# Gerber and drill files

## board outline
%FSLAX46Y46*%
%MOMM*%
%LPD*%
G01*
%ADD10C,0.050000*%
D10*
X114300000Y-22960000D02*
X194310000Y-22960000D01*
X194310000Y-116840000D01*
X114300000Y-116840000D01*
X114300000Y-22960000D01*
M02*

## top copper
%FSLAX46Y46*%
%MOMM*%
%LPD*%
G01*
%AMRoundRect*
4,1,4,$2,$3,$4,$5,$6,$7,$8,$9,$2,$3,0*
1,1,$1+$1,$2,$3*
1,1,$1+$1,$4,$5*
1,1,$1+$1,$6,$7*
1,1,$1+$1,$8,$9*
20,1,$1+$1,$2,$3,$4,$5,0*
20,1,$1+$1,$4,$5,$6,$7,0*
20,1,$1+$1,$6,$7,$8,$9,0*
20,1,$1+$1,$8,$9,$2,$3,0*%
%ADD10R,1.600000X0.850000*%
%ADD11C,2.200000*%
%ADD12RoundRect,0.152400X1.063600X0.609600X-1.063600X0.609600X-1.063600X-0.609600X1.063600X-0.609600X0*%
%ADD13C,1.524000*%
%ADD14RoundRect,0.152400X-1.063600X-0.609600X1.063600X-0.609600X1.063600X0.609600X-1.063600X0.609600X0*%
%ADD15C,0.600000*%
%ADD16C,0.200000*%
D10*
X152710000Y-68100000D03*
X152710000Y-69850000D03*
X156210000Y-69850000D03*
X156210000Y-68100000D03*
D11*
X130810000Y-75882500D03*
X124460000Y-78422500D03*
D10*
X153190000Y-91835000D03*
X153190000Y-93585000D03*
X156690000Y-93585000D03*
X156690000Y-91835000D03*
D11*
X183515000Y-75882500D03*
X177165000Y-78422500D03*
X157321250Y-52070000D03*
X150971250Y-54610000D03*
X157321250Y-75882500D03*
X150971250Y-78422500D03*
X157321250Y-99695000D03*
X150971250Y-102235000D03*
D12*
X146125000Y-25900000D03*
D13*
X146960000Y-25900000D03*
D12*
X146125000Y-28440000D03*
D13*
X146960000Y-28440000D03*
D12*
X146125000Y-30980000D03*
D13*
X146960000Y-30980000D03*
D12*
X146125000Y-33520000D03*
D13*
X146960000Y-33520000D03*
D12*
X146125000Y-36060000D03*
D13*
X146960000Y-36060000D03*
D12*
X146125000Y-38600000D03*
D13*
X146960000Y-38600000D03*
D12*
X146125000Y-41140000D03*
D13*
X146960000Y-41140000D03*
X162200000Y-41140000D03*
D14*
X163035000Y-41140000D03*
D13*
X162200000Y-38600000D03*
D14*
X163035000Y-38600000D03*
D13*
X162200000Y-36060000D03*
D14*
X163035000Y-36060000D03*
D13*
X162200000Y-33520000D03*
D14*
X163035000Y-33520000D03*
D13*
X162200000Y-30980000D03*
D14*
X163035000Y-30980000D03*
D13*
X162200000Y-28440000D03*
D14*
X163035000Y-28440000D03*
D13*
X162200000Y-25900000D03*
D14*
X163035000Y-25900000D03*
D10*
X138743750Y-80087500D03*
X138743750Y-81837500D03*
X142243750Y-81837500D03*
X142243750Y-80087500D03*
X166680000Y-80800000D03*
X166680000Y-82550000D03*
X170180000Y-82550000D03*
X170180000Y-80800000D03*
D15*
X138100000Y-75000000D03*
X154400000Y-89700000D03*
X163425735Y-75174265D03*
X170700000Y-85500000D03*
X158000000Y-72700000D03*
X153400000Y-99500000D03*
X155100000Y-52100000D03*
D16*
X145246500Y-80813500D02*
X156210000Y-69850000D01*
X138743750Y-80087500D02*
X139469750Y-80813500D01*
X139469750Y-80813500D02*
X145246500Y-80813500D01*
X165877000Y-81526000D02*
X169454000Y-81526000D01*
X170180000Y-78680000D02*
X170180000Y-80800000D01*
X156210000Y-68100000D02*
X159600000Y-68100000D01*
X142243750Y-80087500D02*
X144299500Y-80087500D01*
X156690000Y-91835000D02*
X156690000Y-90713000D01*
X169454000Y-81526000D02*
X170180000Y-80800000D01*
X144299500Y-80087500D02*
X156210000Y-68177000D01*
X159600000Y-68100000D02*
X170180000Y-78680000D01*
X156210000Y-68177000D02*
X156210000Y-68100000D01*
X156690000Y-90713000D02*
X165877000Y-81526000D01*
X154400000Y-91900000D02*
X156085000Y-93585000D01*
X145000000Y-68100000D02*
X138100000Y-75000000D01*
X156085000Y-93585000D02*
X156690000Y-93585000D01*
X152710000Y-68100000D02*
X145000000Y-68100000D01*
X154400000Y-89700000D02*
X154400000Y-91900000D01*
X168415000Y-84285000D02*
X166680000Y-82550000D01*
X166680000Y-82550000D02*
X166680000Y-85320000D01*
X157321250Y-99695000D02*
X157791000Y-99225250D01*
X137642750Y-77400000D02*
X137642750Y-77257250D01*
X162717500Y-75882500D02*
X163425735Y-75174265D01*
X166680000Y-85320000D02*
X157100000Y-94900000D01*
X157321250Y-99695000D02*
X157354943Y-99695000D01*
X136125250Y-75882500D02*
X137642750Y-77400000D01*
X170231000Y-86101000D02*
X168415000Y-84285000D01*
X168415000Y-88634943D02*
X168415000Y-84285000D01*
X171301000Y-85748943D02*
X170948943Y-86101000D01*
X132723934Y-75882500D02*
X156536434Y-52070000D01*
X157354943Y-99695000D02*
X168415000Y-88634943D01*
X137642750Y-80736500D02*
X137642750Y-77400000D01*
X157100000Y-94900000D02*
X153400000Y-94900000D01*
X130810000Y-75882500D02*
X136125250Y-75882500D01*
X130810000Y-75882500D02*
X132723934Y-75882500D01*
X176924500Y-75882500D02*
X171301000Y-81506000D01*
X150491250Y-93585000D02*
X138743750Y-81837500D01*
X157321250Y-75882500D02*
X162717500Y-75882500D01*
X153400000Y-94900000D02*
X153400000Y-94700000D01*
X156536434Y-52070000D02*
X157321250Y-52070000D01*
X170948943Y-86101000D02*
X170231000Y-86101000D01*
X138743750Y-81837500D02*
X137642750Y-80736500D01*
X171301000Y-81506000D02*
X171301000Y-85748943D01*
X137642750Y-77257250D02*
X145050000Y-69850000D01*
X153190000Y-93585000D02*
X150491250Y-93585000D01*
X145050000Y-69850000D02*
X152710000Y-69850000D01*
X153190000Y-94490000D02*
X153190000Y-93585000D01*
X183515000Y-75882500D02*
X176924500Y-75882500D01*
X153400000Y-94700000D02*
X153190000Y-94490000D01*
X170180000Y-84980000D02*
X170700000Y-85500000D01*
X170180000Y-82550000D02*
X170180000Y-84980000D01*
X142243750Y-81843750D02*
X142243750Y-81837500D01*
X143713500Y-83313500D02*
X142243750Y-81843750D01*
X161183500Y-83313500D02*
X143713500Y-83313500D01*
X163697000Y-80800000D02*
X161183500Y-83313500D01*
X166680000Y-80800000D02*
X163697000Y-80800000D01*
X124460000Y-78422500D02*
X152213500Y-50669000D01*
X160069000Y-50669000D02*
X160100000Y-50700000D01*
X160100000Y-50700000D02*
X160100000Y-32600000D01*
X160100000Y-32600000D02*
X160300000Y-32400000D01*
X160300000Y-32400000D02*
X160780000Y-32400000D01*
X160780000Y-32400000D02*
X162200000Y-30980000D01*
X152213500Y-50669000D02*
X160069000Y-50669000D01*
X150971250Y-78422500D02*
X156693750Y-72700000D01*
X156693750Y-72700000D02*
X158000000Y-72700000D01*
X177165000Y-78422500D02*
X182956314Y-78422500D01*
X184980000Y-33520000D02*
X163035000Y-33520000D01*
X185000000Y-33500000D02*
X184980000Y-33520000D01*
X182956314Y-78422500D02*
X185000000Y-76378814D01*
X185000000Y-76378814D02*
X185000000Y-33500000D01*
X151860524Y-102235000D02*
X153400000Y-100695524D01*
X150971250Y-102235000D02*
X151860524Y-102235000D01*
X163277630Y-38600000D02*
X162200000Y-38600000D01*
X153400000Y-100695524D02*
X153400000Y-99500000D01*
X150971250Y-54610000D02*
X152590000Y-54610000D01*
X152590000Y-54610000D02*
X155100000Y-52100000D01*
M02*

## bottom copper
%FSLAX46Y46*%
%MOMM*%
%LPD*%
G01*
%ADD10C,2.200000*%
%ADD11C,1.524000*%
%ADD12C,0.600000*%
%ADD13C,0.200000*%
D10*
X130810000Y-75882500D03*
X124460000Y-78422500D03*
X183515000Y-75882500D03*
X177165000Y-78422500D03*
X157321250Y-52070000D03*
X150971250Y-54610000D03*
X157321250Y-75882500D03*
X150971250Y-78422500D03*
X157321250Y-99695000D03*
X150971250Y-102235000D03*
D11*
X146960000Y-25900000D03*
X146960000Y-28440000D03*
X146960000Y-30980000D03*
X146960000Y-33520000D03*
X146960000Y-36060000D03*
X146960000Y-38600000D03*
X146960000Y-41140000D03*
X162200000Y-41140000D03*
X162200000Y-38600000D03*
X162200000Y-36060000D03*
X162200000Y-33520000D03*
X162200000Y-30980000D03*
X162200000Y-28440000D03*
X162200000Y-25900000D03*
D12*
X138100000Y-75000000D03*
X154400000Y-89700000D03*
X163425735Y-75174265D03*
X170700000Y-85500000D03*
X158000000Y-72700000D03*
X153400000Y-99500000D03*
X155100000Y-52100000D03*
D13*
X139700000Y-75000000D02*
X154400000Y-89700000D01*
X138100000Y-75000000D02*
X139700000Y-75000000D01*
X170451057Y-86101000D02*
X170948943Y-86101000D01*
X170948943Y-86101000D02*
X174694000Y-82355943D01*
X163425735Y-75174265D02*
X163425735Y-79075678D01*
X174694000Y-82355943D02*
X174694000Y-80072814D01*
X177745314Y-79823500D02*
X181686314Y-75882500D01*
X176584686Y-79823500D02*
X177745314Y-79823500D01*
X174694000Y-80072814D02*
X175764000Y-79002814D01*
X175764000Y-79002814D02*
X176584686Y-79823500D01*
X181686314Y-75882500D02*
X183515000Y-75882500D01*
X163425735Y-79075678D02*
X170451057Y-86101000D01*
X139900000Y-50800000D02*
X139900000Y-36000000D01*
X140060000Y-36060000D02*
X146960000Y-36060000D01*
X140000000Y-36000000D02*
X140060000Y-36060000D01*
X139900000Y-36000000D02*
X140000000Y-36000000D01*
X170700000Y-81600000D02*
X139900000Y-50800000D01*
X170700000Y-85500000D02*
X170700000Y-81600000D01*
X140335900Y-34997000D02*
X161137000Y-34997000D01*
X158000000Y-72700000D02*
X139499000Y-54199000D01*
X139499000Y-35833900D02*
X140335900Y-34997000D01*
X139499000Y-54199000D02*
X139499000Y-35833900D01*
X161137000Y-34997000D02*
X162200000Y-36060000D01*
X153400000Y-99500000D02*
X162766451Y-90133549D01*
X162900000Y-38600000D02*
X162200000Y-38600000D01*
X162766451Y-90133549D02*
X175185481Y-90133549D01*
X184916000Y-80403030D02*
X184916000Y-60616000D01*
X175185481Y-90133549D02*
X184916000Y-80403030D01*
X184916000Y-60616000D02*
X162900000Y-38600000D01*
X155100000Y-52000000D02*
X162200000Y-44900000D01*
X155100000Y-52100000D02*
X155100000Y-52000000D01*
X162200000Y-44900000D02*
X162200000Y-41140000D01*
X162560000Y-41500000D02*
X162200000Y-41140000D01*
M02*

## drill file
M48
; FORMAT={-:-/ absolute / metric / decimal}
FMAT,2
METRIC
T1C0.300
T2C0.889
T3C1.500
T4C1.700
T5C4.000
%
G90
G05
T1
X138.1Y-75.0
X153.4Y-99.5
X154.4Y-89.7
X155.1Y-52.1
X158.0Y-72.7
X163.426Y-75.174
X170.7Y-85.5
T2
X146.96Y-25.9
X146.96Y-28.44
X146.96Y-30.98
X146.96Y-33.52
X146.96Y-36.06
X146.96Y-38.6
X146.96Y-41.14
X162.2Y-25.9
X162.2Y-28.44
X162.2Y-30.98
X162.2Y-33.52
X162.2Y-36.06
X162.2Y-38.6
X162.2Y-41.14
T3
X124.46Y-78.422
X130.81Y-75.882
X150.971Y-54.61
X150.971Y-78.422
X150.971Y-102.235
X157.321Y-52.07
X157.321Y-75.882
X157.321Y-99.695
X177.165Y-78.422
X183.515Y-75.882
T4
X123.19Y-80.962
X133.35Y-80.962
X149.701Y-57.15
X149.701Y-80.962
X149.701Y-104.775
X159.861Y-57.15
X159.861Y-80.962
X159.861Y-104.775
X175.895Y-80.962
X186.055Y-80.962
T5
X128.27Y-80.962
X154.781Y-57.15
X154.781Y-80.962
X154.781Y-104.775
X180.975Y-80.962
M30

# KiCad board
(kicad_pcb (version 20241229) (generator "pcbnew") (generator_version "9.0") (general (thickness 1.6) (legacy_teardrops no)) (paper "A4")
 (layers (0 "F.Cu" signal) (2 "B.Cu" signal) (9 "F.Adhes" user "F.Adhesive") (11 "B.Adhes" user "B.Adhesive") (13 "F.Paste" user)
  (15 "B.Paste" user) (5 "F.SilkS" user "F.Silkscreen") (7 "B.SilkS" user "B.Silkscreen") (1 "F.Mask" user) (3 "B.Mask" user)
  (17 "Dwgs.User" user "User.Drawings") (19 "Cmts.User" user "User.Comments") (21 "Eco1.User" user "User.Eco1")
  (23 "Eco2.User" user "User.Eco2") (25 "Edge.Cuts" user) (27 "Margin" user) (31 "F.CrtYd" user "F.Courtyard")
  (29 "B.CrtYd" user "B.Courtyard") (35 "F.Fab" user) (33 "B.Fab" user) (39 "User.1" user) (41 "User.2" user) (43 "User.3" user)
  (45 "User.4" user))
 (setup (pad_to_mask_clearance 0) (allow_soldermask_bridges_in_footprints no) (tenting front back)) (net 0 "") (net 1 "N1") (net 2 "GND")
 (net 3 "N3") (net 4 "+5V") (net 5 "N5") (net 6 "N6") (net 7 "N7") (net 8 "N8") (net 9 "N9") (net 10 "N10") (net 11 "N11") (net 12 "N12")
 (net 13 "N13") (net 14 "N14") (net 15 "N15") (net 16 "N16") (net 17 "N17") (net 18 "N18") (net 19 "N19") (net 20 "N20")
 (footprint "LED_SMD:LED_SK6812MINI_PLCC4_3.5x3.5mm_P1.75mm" (layer "F.Cu") (at 154.46 68.975)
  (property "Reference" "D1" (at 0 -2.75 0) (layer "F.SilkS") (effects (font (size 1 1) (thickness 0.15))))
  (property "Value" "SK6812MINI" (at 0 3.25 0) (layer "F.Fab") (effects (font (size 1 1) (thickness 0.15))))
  (pad "1" smd rect (at -1.75 -0.875) (size 1.6 0.85) (layers "F.Cu" "F.Mask" "F.Paste") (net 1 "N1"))
  (pad "2" smd rect (at -1.75 0.875) (size 1.6 0.85) (layers "F.Cu" "F.Mask" "F.Paste") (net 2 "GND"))
  (pad "3" smd rect (at 1.75 0.875) (size 1.6 0.85) (layers "F.Cu" "F.Mask" "F.Paste") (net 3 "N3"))
  (pad "4" smd rect (at 1.75 -0.875) (size 1.6 0.85) (layers "F.Cu" "F.Mask" "F.Paste") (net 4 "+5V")))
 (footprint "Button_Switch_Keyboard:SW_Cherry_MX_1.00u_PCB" (layer "F.Cu") (at 130.81 75.8825)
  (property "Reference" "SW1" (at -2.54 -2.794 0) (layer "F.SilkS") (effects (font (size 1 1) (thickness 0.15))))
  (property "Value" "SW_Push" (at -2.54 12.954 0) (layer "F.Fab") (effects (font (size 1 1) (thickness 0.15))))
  (pad "" np_thru_hole circle (at -7.62 5.08) (size 1.7 1.7) (drill 1.7) (layers "*.Cu" "*.Mask"))
  (pad "" np_thru_hole circle (at -2.54 5.08) (size 4 4) (drill 4) (layers "*.Cu" "*.Mask"))
  (pad "" np_thru_hole circle (at 2.54 5.08) (size 1.7 1.7) (drill 1.7) (layers "*.Cu" "*.Mask"))
  (pad "1" thru_hole circle (at 0 0) (size 2.2 2.2) (drill 1.5) (layers "*.Cu" "*.Mask") (remove_unused_layers no) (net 2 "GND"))
  (pad "2" thru_hole circle (at -6.35 2.54) (size 2.2 2.2) (drill 1.5) (layers "*.Cu" "*.Mask") (remove_unused_layers no) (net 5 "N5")))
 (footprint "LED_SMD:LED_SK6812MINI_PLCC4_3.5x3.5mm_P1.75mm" (layer "F.Cu") (at 154.94 92.71)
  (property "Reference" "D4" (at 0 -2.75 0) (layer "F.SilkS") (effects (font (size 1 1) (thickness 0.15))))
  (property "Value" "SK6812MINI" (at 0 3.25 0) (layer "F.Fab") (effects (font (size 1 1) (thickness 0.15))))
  (pad "1" smd rect (at -1.75 -0.875) (size 1.6 0.85) (layers "F.Cu" "F.Mask" "F.Paste") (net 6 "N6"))
  (pad "2" smd rect (at -1.75 0.875) (size 1.6 0.85) (layers "F.Cu" "F.Mask" "F.Paste") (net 2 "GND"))
  (pad "3" smd rect (at 1.75 0.875) (size 1.6 0.85) (layers "F.Cu" "F.Mask" "F.Paste") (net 1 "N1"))
  (pad "4" smd rect (at 1.75 -0.875) (size 1.6 0.85) (layers "F.Cu" "F.Mask" "F.Paste") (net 4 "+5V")))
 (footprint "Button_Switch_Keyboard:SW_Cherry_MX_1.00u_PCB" (layer "F.Cu") (at 183.515 75.8825)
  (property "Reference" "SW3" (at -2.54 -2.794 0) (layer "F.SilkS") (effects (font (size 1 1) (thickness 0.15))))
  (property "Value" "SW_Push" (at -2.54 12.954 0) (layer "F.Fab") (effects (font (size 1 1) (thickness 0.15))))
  (pad "" np_thru_hole circle (at -7.62 5.08) (size 1.7 1.7) (drill 1.7) (layers "*.Cu" "*.Mask"))
  (pad "" np_thru_hole circle (at -2.54 5.08) (size 4 4) (drill 4) (layers "*.Cu" "*.Mask"))
  (pad "" np_thru_hole circle (at 2.54 5.08) (size 1.7 1.7) (drill 1.7) (layers "*.Cu" "*.Mask"))
  (pad "1" thru_hole circle (at 0 0) (size 2.2 2.2) (drill 1.5) (layers "*.Cu" "*.Mask") (remove_unused_layers no) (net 2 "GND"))
  (pad "2" thru_hole circle (at -6.35 2.54) (size 2.2 2.2) (drill 1.5) (layers "*.Cu" "*.Mask") (remove_unused_layers no) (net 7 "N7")))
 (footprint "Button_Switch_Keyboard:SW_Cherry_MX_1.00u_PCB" (layer "F.Cu") (at 157.32125 52.07)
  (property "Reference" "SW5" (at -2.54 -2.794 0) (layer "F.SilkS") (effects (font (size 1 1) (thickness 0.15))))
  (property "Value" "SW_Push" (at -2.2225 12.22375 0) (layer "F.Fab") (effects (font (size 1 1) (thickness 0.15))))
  (pad "" np_thru_hole circle (at -7.62 5.08) (size 1.7 1.7) (drill 1.7) (layers "*.Cu" "*.Mask"))
  (pad "" np_thru_hole circle (at -2.54 5.08) (size 4 4) (drill 4) (layers "*.Cu" "*.Mask"))
  (pad "" np_thru_hole circle (at 2.54 5.08) (size 1.7 1.7) (drill 1.7) (layers "*.Cu" "*.Mask"))
  (pad "1" thru_hole circle (at 0 0) (size 2.2 2.2) (drill 1.5) (layers "*.Cu" "*.Mask") (remove_unused_layers no) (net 2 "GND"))
  (pad "2" thru_hole circle (at -6.35 2.54) (size 2.2 2.2) (drill 1.5) (layers "*.Cu" "*.Mask") (remove_unused_layers no) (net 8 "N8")))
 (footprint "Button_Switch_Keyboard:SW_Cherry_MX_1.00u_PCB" (layer "F.Cu") (at 157.32125 75.8825)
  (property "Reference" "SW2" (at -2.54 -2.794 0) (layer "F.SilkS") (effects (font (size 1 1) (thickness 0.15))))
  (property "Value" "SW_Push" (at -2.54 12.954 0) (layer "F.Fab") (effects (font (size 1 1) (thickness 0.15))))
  (pad "" np_thru_hole circle (at -7.62 5.08) (size 1.7 1.7) (drill 1.7) (layers "*.Cu" "*.Mask"))
  (pad "" np_thru_hole circle (at -2.54 5.08) (size 4 4) (drill 4) (layers "*.Cu" "*.Mask"))
  (pad "" np_thru_hole circle (at 2.54 5.08) (size 1.7 1.7) (drill 1.7) (layers "*.Cu" "*.Mask"))
  (pad "1" thru_hole circle (at 0 0) (size 2.2 2.2) (drill 1.5) (layers "*.Cu" "*.Mask") (remove_unused_layers no) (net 2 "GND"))
  (pad "2" thru_hole circle (at -6.35 2.54) (size 2.2 2.2) (drill 1.5) (layers "*.Cu" "*.Mask") (remove_unused_layers no) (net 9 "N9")))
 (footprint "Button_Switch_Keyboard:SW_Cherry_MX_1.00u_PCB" (layer "F.Cu") (at 157.32125 99.695)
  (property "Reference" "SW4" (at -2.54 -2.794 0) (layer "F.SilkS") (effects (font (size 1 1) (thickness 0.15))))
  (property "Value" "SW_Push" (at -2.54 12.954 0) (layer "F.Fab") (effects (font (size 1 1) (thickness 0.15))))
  (pad "" np_thru_hole circle (at -7.62 5.08) (size 1.7 1.7) (drill 1.7) (layers "*.Cu" "*.Mask"))
  (pad "" np_thru_hole circle (at -2.54 5.08) (size 4 4) (drill 4) (layers "*.Cu" "*.Mask"))
  (pad "" np_thru_hole circle (at 2.54 5.08) (size 1.7 1.7) (drill 1.7) (layers "*.Cu" "*.Mask"))
  (pad "1" thru_hole circle (at 0 0) (size 2.2 2.2) (drill 1.5) (layers "*.Cu" "*.Mask") (remove_unused_layers no) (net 2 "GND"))
  (pad "2" thru_hole circle (at -6.35 2.54) (size 2.2 2.2) (drill 1.5) (layers "*.Cu" "*.Mask") (remove_unused_layers no) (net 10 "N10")))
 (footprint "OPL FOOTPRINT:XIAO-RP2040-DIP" (layer "F.Cu") (at 154.58 33.52)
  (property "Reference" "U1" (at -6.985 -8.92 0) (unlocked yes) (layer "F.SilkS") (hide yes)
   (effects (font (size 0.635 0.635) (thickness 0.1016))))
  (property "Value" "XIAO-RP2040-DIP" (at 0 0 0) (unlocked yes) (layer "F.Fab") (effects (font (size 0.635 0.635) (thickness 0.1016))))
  (pad "1" smd roundrect (at -8.455 -7.62 180) (size 2.432 1.524) (layers "F.Cu" "F.Mask") (roundrect_rratio 0.1) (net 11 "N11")
   (thermal_bridge_angle 45))
  (pad "1" thru_hole circle (at -7.62 -7.62 180) (size 1.524 1.524) (drill 0.889) (layers "*.Cu" "*.Mask") (remove_unused_layers no)
   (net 11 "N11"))
  (pad "2" smd roundrect (at -8.455 -5.08 180) (size 2.432 1.524) (layers "F.Cu" "F.Mask") (roundrect_rratio 0.1) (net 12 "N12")
   (thermal_bridge_angle 45))
  (pad "2" thru_hole circle (at -7.62 -5.08 180) (size 1.524 1.524) (drill 0.889) (layers "*.Cu" "*.Mask") (remove_unused_layers no)
   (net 12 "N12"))
  (pad "3" smd roundrect (at -8.455 -2.54 180) (size 2.432 1.524) (layers "F.Cu" "F.Mask") (roundrect_rratio 0.1) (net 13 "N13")
   (thermal_bridge_angle 45))
  (pad "3" thru_hole circle (at -7.62 -2.54 180) (size 1.524 1.524) (drill 0.889) (layers "*.Cu" "*.Mask") (remove_unused_layers no)
   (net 13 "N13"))
  (pad "4" smd roundrect (at -8.455 0 180) (size 2.432 1.524) (layers "F.Cu" "F.Mask") (roundrect_rratio 0.1) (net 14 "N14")
   (thermal_bridge_angle 45))
  (pad "4" thru_hole circle (at -7.62 0 180) (size 1.524 1.524) (drill 0.889) (layers "*.Cu" "*.Mask") (remove_unused_layers no)
   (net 14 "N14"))
  (pad "5" smd roundrect (at -8.455 2.54 180) (size 2.432 1.524) (layers "F.Cu" "F.Mask") (roundrect_rratio 0.1) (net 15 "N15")
   (thermal_bridge_angle 45))
  (pad "5" thru_hole circle (at -7.62 2.54 180) (size 1.524 1.524) (drill 0.889) (layers "*.Cu" "*.Mask") (remove_unused_layers no)
   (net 15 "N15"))
  (pad "6" smd roundrect (at -8.455 5.08 180) (size 2.432 1.524) (layers "F.Cu" "F.Mask") (roundrect_rratio 0.1) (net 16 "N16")
   (thermal_bridge_angle 45))
  (pad "6" thru_hole circle (at -7.62 5.08 180) (size 1.524 1.524) (drill 0.889) (layers "*.Cu" "*.Mask") (remove_unused_layers no)
   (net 16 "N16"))
  (pad "7" smd roundrect (at -8.455 7.62 180) (size 2.432 1.524) (layers "F.Cu" "F.Mask") (roundrect_rratio 0.1) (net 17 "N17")
   (thermal_bridge_angle 45))
  (pad "7" thru_hole circle (at -7.62 7.62 180) (size 1.524 1.524) (drill 0.889) (layers "*.Cu" "*.Mask") (remove_unused_layers no)
   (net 17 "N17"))
  (pad "8" thru_hole circle (at 7.62 7.62) (size 1.524 1.524) (drill 0.889) (layers "*.Cu" "*.Mask") (remove_unused_layers no) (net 8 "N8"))
  (pad "8" smd roundrect (at 8.455 7.62) (size 2.432 1.524) (layers "F.Cu" "F.Mask") (roundrect_rratio 0.1) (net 8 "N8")
   (thermal_bridge_angle 45))
  (pad "9" thru_hole circle (at 7.62 5.08) (size 1.524 1.524) (drill 0.889) (layers "*.Cu" "*.Mask") (remove_unused_layers no)
   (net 10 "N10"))
  (pad "9" smd roundrect (at 8.455 5.08) (size 2.432 1.524) (layers "F.Cu" "F.Mask") (roundrect_rratio 0.1) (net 10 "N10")
   (thermal_bridge_angle 45))
  (pad "10" thru_hole circle (at 7.62 2.54) (size 1.524 1.524) (drill 0.889) (layers "*.Cu" "*.Mask") (remove_unused_layers no) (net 9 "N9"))
  (pad "10" smd roundrect (at 8.455 2.54) (size 2.432 1.524) (layers "F.Cu" "F.Mask") (roundrect_rratio 0.1) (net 9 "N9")
   (thermal_bridge_angle 45))
  (pad "11" thru_hole circle (at 7.62 0) (size 1.524 1.524) (drill 0.889) (layers "*.Cu" "*.Mask") (remove_unused_layers no) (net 7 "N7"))
  (pad "11" smd roundrect (at 8.455 0) (size 2.432 1.524) (layers "F.Cu" "F.Mask") (roundrect_rratio 0.1) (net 7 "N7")
   (thermal_bridge_angle 45))
  (pad "12" thru_hole circle (at 7.62 -2.54) (size 1.524 1.524) (drill 0.889) (layers "*.Cu" "*.Mask") (remove_unused_layers no)
   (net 5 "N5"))
  (pad "12" smd roundrect (at 8.455 -2.54) (size 2.432 1.524) (layers "F.Cu" "F.Mask") (roundrect_rratio 0.1) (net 5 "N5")
   (thermal_bridge_angle 45))
  (pad "13" thru_hole circle (at 7.62 -5.08) (size 1.524 1.524) (drill 0.889) (layers "*.Cu" "*.Mask") (remove_unused_layers no)
   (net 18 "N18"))
  (pad "13" smd roundrect (at 8.455 -5.08) (size 2.432 1.524) (layers "F.Cu" "F.Mask") (roundrect_rratio 0.1) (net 18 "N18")
   (thermal_bridge_angle 45))
  (pad "14" thru_hole circle (at 7.62 -7.62) (size 1.524 1.524) (drill 0.889) (layers "*.Cu" "*.Mask") (remove_unused_layers no)
   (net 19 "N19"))
  (pad "14" smd roundrect (at 8.455 -7.62) (size 2.432 1.524) (layers "F.Cu" "F.Mask") (roundrect_rratio 0.1) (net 19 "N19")
   (thermal_bridge_angle 45)))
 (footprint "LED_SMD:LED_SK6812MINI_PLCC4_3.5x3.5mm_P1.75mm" (layer "F.Cu") (at 140.49375 80.9625)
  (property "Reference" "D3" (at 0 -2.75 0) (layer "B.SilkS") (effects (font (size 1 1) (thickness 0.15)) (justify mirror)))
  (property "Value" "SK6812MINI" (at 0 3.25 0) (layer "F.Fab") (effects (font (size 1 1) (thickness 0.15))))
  (pad "1" smd rect (at -1.75 -0.875) (size 1.6 0.85) (layers "F.Cu" "F.Mask" "F.Paste") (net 3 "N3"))
  (pad "2" smd rect (at -1.75 0.875) (size 1.6 0.85) (layers "F.Cu" "F.Mask" "F.Paste") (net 2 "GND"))
  (pad "3" smd rect (at 1.75 0.875) (size 1.6 0.85) (layers "F.Cu" "F.Mask" "F.Paste") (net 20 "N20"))
  (pad "4" smd rect (at 1.75 -0.875) (size 1.6 0.85) (layers "F.Cu" "F.Mask" "F.Paste") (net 4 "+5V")))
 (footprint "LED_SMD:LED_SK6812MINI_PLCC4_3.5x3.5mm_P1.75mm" (layer "F.Cu") (at 168.43 81.675)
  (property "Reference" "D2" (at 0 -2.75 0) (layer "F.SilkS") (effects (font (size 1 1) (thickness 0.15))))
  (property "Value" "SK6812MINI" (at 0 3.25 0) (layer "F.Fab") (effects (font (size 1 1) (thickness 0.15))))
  (pad "1" smd rect (at -1.75 -0.875) (size 1.6 0.85) (layers "F.Cu" "F.Mask" "F.Paste") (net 20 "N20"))
  (pad "2" smd rect (at -1.75 0.875) (size 1.6 0.85) (layers "F.Cu" "F.Mask" "F.Paste") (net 2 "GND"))
  (pad "3" smd rect (at 1.75 0.875) (size 1.6 0.85) (layers "F.Cu" "F.Mask" "F.Paste") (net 15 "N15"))
  (pad "4" smd rect (at 1.75 -0.875) (size 1.6 0.85) (layers "F.Cu" "F.Mask" "F.Paste") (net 4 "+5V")))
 (gr_rect (start 114.3 22.96) (end 194.31 116.84) (stroke (width 0.05) (type default)) (fill no) (layer "Edge.Cuts"))
 (segment (start 145.2465 80.8135) (end 156.21 69.85) (width 0.2) (layer "F.Cu") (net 3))
 (segment (start 138.74375 80.0875) (end 139.46975 80.8135) (width 0.2) (layer "F.Cu") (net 3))
 (segment (start 139.46975 80.8135) (end 145.2465 80.8135) (width 0.2) (layer "F.Cu") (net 3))
 (segment (start 165.877 81.526) (end 169.454 81.526) (width 0.2) (layer "F.Cu") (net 4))
 (segment (start 170.18 78.68) (end 170.18 80.8) (width 0.2) (layer "F.Cu") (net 4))
 (segment (start 156.21 68.1) (end 159.6 68.1) (width 0.2) (layer "F.Cu") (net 4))
 (segment (start 142.24375 80.0875) (end 144.2995 80.0875) (width 0.2) (layer "F.Cu") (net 4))
 (segment (start 156.69 91.835) (end 156.69 90.713) (width 0.2) (layer "F.Cu") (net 4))
 (segment (start 169.454 81.526) (end 170.18 80.8) (width 0.2) (layer "F.Cu") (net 4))
 (segment (start 144.2995 80.0875) (end 156.21 68.177) (width 0.2) (layer "F.Cu") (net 4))
 (segment (start 159.6 68.1) (end 170.18 78.68) (width 0.2) (layer "F.Cu") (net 4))
 (segment (start 156.21 68.177) (end 156.21 68.1) (width 0.2) (layer "F.Cu") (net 4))
 (segment (start 156.69 90.713) (end 165.877 81.526) (width 0.2) (layer "F.Cu") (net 4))
 (segment (start 154.4 91.9) (end 156.085 93.585) (width 0.2) (layer "F.Cu") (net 1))
 (segment (start 145 68.1) (end 138.1 75) (width 0.2) (layer "F.Cu") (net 1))
 (segment (start 156.085 93.585) (end 156.69 93.585) (width 0.2) (layer "F.Cu") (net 1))
 (segment (start 152.71 68.1) (end 145 68.1) (width 0.2) (layer "F.Cu") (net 1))
 (segment (start 154.4 89.7) (end 154.4 91.9) (width 0.2) (layer "F.Cu") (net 1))
 (via (at 138.1 75) (size 0.6) (drill 0.3) (layers "F.Cu" "B.Cu") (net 1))
 (via (at 154.4 89.7) (size 0.6) (drill 0.3) (layers "F.Cu" "B.Cu") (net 1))
 (segment (start 139.7 75) (end 154.4 89.7) (width 0.2) (layer "B.Cu") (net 1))
 (segment (start 138.1 75) (end 139.7 75) (width 0.2) (layer "B.Cu") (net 1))
 (segment (start 168.415 84.285) (end 166.68 82.55) (width 0.2) (layer "F.Cu") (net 2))
 (segment (start 166.68 82.55) (end 166.68 85.32) (width 0.2) (layer "F.Cu") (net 2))
 (segment (start 157.32125 99.695) (end 157.791 99.22525) (width 0.2) (layer "F.Cu") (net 2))
 (segment (start 137.64275 77.4) (end 137.64275 77.25725) (width 0.2) (layer "F.Cu") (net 2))
 (segment (start 162.7175 75.8825) (end 163.425735 75.174265) (width 0.2) (layer "F.Cu") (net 2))
 (segment (start 166.68 85.32) (end 157.1 94.9) (width 0.2) (layer "F.Cu") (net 2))
 (segment (start 157.32125 99.695) (end 157.354943 99.695) (width 0.2) (layer "F.Cu") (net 2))
 (segment (start 136.12525 75.8825) (end 137.64275 77.4) (width 0.2) (layer "F.Cu") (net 2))
 (segment (start 170.231 86.101) (end 168.415 84.285) (width 0.2) (layer "F.Cu") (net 2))
 (segment (start 168.415 88.634943) (end 168.415 84.285) (width 0.2) (layer "F.Cu") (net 2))
 (segment (start 171.301 85.748943) (end 170.948943 86.101) (width 0.2) (layer "F.Cu") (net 2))
 (segment (start 132.723934 75.8825) (end 156.536434 52.07) (width 0.2) (layer "F.Cu") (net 2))
 (segment (start 157.354943 99.695) (end 168.415 88.634943) (width 0.2) (layer "F.Cu") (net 2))
 (segment (start 137.64275 80.7365) (end 137.64275 77.4) (width 0.2) (layer "F.Cu") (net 2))
 (segment (start 157.1 94.9) (end 153.4 94.9) (width 0.2) (layer "F.Cu") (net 2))
 (segment (start 130.81 75.8825) (end 136.12525 75.8825) (width 0.2) (layer "F.Cu") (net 2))
 (segment (start 130.81 75.8825) (end 132.723934 75.8825) (width 0.2) (layer "F.Cu") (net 2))
 (segment (start 176.9245 75.8825) (end 171.301 81.506) (width 0.2) (layer "F.Cu") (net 2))
 (segment (start 150.49125 93.585) (end 138.74375 81.8375) (width 0.2) (layer "F.Cu") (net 2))
 (segment (start 157.32125 75.8825) (end 162.7175 75.8825) (width 0.2) (layer "F.Cu") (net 2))
 (segment (start 153.4 94.9) (end 153.4 94.7) (width 0.2) (layer "F.Cu") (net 2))
 (segment (start 156.536434 52.07) (end 157.32125 52.07) (width 0.2) (layer "F.Cu") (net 2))
 (segment (start 170.948943 86.101) (end 170.231 86.101) (width 0.2) (layer "F.Cu") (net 2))
 (segment (start 138.74375 81.8375) (end 137.64275 80.7365) (width 0.2) (layer "F.Cu") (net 2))
 (segment (start 171.301 81.506) (end 171.301 85.748943) (width 0.2) (layer "F.Cu") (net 2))
 (segment (start 137.64275 77.25725) (end 145.05 69.85) (width 0.2) (layer "F.Cu") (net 2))
 (segment (start 153.19 93.585) (end 150.49125 93.585) (width 0.2) (layer "F.Cu") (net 2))
 (segment (start 145.05 69.85) (end 152.71 69.85) (width 0.2) (layer "F.Cu") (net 2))
 (segment (start 153.19 94.49) (end 153.19 93.585) (width 0.2) (layer "F.Cu") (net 2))
 (segment (start 183.515 75.8825) (end 176.9245 75.8825) (width 0.2) (layer "F.Cu") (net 2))
 (segment (start 153.4 94.7) (end 153.19 94.49) (width 0.2) (layer "F.Cu") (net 2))
 (via (at 163.425735 75.174265) (size 0.6) (drill 0.3) (layers "F.Cu" "B.Cu") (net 2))
 (segment (start 170.451057 86.101) (end 170.948943 86.101) (width 0.2) (layer "B.Cu") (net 2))
 (segment (start 170.948943 86.101) (end 174.694 82.355943) (width 0.2) (layer "B.Cu") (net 2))
 (segment (start 163.425735 75.174265) (end 163.425735 79.075678) (width 0.2) (layer "B.Cu") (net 2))
 (segment (start 174.694 82.355943) (end 174.694 80.072814) (width 0.2) (layer "B.Cu") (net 2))
 (segment (start 177.745314 79.8235) (end 181.686314 75.8825) (width 0.2) (layer "B.Cu") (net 2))
 (segment (start 176.584686 79.8235) (end 177.745314 79.8235) (width 0.2) (layer "B.Cu") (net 2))
 (segment (start 174.694 80.072814) (end 175.764 79.002814) (width 0.2) (layer "B.Cu") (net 2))
 (segment (start 175.764 79.002814) (end 176.584686 79.8235) (width 0.2) (layer "B.Cu") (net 2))
 (segment (start 181.686314 75.8825) (end 183.515 75.8825) (width 0.2) (layer "B.Cu") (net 2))
 (segment (start 163.425735 79.075678) (end 170.451057 86.101) (width 0.2) (layer "B.Cu") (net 2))
 (segment (start 170.18 84.98) (end 170.7 85.5) (width 0.2) (layer "F.Cu") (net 15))
 (segment (start 170.18 82.55) (end 170.18 84.98) (width 0.2) (layer "F.Cu") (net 15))
 (via (at 170.7 85.5) (size 0.6) (drill 0.3) (layers "F.Cu" "B.Cu") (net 15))
 (segment (start 139.9 50.8) (end 139.9 36) (width 0.2) (layer "B.Cu") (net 15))
 (segment (start 140.06 36.06) (end 146.96 36.06) (width 0.2) (layer "B.Cu") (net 15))
 (segment (start 140 36) (end 140.06 36.06) (width 0.2) (layer "B.Cu") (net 15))
 (segment (start 139.9 36) (end 140 36) (width 0.2) (layer "B.Cu") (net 15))
 (segment (start 170.7 81.6) (end 139.9 50.8) (width 0.2) (layer "B.Cu") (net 15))
 (segment (start 170.7 85.5) (end 170.7 81.6) (width 0.2) (layer "B.Cu") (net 15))
 (segment (start 142.24375 81.84375) (end 142.24375 81.8375) (width 0.2) (layer "F.Cu") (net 20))
 (segment (start 143.7135 83.3135) (end 142.24375 81.84375) (width 0.2) (layer "F.Cu") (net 20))
 (segment (start 161.1835 83.3135) (end 143.7135 83.3135) (width 0.2) (layer "F.Cu") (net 20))
 (segment (start 163.697 80.8) (end 161.1835 83.3135) (width 0.2) (layer "F.Cu") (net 20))
 (segment (start 166.68 80.8) (end 163.697 80.8) (width 0.2) (layer "F.Cu") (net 20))
 (segment (start 124.46 78.4225) (end 152.2135 50.669) (width 0.2) (layer "F.Cu") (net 5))
 (segment (start 160.069 50.669) (end 160.1 50.7) (width 0.2) (layer "F.Cu") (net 5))
 (segment (start 160.1 50.7) (end 160.1 32.6) (width 0.2) (layer "F.Cu") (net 5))
 (segment (start 160.1 32.6) (end 160.3 32.4) (width 0.2) (layer "F.Cu") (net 5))
 (segment (start 160.3 32.4) (end 160.78 32.4) (width 0.2) (layer "F.Cu") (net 5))
 (segment (start 160.78 32.4) (end 162.2 30.98) (width 0.2) (layer "F.Cu") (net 5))
 (segment (start 152.2135 50.669) (end 160.069 50.669) (width 0.2) (layer "F.Cu") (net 5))
 (segment (start 150.97125 78.4225) (end 156.69375 72.7) (width 0.2) (layer "F.Cu") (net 9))
 (segment (start 156.69375 72.7) (end 158 72.7) (width 0.2) (layer "F.Cu") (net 9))
 (via (at 158 72.7) (size 0.6) (drill 0.3) (layers "F.Cu" "B.Cu") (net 9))
 (segment (start 140.3359 34.997) (end 161.137 34.997) (width 0.2) (layer "B.Cu") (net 9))
 (segment (start 158 72.7) (end 139.499 54.199) (width 0.2) (layer "B.Cu") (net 9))
 (segment (start 139.499 35.8339) (end 140.3359 34.997) (width 0.2) (layer "B.Cu") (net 9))
 (segment (start 139.499 54.199) (end 139.499 35.8339) (width 0.2) (layer "B.Cu") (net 9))
 (segment (start 161.137 34.997) (end 162.2 36.06) (width 0.2) (layer "B.Cu") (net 9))
 (segment (start 177.165 78.4225) (end 182.956314 78.4225) (width 0.2) (layer "F.Cu") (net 7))
 (segment (start 184.98 33.52) (end 163.035 33.52) (width 0.2) (layer "F.Cu") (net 7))
 (segment (start 185 33.5) (end 184.98 33.52) (width 0.2) (layer "F.Cu") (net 7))
 (segment (start 182.956314 78.4225) (end 185 76.378814) (width 0.2) (layer "F.Cu") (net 7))
 (segment (start 185 76.378814) (end 185 33.5) (width 0.2) (layer "F.Cu") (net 7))
 (segment (start 151.860524 102.235) (end 153.4 100.695524) (width 0.2) (layer "F.Cu") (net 10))
 (segment (start 150.97125 102.235) (end 151.860524 102.235) (width 0.2) (layer "F.Cu") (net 10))
 (segment (start 163.27763 38.6) (end 162.2 38.6) (width 0.2) (layer "F.Cu") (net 10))
 (segment (start 153.4 100.695524) (end 153.4 99.5) (width 0.2) (layer "F.Cu") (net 10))
 (via (at 153.4 99.5) (size 0.6) (drill 0.3) (layers "F.Cu" "B.Cu") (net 10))
 (segment (start 153.4 99.5) (end 162.766451 90.133549) (width 0.2) (layer "B.Cu") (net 10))
 (segment (start 162.9 38.6) (end 162.2 38.6) (width 0.2) (layer "B.Cu") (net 10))
 (segment (start 162.766451 90.133549) (end 175.185481 90.133549) (width 0.2) (layer "B.Cu") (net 10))
 (segment (start 184.916 80.40303) (end 184.916 60.616) (width 0.2) (layer "B.Cu") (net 10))
 (segment (start 175.185481 90.133549) (end 184.916 80.40303) (width 0.2) (layer "B.Cu") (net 10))
 (segment (start 184.916 60.616) (end 162.9 38.6) (width 0.2) (layer "B.Cu") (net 10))
 (segment (start 150.97125 54.61) (end 152.59 54.61) (width 0.2) (layer "F.Cu") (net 8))
 (segment (start 152.59 54.61) (end 155.1 52.1) (width 0.2) (layer "F.Cu") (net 8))
 (via (at 155.1 52.1) (size 0.6) (drill 0.3) (layers "F.Cu" "B.Cu") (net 8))
 (segment (start 155.1 52) (end 162.2 44.9) (width 0.2) (layer "B.Cu") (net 8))
 (segment (start 155.1 52.1) (end 155.1 52) (width 0.2) (layer "B.Cu") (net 8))
 (segment (start 162.2 44.9) (end 162.2 41.14) (width 0.2) (layer "B.Cu") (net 8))
 (segment (start 162.56 41.5) (end 162.2 41.14) (width 0.2) (layer "B.Cu") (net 8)))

